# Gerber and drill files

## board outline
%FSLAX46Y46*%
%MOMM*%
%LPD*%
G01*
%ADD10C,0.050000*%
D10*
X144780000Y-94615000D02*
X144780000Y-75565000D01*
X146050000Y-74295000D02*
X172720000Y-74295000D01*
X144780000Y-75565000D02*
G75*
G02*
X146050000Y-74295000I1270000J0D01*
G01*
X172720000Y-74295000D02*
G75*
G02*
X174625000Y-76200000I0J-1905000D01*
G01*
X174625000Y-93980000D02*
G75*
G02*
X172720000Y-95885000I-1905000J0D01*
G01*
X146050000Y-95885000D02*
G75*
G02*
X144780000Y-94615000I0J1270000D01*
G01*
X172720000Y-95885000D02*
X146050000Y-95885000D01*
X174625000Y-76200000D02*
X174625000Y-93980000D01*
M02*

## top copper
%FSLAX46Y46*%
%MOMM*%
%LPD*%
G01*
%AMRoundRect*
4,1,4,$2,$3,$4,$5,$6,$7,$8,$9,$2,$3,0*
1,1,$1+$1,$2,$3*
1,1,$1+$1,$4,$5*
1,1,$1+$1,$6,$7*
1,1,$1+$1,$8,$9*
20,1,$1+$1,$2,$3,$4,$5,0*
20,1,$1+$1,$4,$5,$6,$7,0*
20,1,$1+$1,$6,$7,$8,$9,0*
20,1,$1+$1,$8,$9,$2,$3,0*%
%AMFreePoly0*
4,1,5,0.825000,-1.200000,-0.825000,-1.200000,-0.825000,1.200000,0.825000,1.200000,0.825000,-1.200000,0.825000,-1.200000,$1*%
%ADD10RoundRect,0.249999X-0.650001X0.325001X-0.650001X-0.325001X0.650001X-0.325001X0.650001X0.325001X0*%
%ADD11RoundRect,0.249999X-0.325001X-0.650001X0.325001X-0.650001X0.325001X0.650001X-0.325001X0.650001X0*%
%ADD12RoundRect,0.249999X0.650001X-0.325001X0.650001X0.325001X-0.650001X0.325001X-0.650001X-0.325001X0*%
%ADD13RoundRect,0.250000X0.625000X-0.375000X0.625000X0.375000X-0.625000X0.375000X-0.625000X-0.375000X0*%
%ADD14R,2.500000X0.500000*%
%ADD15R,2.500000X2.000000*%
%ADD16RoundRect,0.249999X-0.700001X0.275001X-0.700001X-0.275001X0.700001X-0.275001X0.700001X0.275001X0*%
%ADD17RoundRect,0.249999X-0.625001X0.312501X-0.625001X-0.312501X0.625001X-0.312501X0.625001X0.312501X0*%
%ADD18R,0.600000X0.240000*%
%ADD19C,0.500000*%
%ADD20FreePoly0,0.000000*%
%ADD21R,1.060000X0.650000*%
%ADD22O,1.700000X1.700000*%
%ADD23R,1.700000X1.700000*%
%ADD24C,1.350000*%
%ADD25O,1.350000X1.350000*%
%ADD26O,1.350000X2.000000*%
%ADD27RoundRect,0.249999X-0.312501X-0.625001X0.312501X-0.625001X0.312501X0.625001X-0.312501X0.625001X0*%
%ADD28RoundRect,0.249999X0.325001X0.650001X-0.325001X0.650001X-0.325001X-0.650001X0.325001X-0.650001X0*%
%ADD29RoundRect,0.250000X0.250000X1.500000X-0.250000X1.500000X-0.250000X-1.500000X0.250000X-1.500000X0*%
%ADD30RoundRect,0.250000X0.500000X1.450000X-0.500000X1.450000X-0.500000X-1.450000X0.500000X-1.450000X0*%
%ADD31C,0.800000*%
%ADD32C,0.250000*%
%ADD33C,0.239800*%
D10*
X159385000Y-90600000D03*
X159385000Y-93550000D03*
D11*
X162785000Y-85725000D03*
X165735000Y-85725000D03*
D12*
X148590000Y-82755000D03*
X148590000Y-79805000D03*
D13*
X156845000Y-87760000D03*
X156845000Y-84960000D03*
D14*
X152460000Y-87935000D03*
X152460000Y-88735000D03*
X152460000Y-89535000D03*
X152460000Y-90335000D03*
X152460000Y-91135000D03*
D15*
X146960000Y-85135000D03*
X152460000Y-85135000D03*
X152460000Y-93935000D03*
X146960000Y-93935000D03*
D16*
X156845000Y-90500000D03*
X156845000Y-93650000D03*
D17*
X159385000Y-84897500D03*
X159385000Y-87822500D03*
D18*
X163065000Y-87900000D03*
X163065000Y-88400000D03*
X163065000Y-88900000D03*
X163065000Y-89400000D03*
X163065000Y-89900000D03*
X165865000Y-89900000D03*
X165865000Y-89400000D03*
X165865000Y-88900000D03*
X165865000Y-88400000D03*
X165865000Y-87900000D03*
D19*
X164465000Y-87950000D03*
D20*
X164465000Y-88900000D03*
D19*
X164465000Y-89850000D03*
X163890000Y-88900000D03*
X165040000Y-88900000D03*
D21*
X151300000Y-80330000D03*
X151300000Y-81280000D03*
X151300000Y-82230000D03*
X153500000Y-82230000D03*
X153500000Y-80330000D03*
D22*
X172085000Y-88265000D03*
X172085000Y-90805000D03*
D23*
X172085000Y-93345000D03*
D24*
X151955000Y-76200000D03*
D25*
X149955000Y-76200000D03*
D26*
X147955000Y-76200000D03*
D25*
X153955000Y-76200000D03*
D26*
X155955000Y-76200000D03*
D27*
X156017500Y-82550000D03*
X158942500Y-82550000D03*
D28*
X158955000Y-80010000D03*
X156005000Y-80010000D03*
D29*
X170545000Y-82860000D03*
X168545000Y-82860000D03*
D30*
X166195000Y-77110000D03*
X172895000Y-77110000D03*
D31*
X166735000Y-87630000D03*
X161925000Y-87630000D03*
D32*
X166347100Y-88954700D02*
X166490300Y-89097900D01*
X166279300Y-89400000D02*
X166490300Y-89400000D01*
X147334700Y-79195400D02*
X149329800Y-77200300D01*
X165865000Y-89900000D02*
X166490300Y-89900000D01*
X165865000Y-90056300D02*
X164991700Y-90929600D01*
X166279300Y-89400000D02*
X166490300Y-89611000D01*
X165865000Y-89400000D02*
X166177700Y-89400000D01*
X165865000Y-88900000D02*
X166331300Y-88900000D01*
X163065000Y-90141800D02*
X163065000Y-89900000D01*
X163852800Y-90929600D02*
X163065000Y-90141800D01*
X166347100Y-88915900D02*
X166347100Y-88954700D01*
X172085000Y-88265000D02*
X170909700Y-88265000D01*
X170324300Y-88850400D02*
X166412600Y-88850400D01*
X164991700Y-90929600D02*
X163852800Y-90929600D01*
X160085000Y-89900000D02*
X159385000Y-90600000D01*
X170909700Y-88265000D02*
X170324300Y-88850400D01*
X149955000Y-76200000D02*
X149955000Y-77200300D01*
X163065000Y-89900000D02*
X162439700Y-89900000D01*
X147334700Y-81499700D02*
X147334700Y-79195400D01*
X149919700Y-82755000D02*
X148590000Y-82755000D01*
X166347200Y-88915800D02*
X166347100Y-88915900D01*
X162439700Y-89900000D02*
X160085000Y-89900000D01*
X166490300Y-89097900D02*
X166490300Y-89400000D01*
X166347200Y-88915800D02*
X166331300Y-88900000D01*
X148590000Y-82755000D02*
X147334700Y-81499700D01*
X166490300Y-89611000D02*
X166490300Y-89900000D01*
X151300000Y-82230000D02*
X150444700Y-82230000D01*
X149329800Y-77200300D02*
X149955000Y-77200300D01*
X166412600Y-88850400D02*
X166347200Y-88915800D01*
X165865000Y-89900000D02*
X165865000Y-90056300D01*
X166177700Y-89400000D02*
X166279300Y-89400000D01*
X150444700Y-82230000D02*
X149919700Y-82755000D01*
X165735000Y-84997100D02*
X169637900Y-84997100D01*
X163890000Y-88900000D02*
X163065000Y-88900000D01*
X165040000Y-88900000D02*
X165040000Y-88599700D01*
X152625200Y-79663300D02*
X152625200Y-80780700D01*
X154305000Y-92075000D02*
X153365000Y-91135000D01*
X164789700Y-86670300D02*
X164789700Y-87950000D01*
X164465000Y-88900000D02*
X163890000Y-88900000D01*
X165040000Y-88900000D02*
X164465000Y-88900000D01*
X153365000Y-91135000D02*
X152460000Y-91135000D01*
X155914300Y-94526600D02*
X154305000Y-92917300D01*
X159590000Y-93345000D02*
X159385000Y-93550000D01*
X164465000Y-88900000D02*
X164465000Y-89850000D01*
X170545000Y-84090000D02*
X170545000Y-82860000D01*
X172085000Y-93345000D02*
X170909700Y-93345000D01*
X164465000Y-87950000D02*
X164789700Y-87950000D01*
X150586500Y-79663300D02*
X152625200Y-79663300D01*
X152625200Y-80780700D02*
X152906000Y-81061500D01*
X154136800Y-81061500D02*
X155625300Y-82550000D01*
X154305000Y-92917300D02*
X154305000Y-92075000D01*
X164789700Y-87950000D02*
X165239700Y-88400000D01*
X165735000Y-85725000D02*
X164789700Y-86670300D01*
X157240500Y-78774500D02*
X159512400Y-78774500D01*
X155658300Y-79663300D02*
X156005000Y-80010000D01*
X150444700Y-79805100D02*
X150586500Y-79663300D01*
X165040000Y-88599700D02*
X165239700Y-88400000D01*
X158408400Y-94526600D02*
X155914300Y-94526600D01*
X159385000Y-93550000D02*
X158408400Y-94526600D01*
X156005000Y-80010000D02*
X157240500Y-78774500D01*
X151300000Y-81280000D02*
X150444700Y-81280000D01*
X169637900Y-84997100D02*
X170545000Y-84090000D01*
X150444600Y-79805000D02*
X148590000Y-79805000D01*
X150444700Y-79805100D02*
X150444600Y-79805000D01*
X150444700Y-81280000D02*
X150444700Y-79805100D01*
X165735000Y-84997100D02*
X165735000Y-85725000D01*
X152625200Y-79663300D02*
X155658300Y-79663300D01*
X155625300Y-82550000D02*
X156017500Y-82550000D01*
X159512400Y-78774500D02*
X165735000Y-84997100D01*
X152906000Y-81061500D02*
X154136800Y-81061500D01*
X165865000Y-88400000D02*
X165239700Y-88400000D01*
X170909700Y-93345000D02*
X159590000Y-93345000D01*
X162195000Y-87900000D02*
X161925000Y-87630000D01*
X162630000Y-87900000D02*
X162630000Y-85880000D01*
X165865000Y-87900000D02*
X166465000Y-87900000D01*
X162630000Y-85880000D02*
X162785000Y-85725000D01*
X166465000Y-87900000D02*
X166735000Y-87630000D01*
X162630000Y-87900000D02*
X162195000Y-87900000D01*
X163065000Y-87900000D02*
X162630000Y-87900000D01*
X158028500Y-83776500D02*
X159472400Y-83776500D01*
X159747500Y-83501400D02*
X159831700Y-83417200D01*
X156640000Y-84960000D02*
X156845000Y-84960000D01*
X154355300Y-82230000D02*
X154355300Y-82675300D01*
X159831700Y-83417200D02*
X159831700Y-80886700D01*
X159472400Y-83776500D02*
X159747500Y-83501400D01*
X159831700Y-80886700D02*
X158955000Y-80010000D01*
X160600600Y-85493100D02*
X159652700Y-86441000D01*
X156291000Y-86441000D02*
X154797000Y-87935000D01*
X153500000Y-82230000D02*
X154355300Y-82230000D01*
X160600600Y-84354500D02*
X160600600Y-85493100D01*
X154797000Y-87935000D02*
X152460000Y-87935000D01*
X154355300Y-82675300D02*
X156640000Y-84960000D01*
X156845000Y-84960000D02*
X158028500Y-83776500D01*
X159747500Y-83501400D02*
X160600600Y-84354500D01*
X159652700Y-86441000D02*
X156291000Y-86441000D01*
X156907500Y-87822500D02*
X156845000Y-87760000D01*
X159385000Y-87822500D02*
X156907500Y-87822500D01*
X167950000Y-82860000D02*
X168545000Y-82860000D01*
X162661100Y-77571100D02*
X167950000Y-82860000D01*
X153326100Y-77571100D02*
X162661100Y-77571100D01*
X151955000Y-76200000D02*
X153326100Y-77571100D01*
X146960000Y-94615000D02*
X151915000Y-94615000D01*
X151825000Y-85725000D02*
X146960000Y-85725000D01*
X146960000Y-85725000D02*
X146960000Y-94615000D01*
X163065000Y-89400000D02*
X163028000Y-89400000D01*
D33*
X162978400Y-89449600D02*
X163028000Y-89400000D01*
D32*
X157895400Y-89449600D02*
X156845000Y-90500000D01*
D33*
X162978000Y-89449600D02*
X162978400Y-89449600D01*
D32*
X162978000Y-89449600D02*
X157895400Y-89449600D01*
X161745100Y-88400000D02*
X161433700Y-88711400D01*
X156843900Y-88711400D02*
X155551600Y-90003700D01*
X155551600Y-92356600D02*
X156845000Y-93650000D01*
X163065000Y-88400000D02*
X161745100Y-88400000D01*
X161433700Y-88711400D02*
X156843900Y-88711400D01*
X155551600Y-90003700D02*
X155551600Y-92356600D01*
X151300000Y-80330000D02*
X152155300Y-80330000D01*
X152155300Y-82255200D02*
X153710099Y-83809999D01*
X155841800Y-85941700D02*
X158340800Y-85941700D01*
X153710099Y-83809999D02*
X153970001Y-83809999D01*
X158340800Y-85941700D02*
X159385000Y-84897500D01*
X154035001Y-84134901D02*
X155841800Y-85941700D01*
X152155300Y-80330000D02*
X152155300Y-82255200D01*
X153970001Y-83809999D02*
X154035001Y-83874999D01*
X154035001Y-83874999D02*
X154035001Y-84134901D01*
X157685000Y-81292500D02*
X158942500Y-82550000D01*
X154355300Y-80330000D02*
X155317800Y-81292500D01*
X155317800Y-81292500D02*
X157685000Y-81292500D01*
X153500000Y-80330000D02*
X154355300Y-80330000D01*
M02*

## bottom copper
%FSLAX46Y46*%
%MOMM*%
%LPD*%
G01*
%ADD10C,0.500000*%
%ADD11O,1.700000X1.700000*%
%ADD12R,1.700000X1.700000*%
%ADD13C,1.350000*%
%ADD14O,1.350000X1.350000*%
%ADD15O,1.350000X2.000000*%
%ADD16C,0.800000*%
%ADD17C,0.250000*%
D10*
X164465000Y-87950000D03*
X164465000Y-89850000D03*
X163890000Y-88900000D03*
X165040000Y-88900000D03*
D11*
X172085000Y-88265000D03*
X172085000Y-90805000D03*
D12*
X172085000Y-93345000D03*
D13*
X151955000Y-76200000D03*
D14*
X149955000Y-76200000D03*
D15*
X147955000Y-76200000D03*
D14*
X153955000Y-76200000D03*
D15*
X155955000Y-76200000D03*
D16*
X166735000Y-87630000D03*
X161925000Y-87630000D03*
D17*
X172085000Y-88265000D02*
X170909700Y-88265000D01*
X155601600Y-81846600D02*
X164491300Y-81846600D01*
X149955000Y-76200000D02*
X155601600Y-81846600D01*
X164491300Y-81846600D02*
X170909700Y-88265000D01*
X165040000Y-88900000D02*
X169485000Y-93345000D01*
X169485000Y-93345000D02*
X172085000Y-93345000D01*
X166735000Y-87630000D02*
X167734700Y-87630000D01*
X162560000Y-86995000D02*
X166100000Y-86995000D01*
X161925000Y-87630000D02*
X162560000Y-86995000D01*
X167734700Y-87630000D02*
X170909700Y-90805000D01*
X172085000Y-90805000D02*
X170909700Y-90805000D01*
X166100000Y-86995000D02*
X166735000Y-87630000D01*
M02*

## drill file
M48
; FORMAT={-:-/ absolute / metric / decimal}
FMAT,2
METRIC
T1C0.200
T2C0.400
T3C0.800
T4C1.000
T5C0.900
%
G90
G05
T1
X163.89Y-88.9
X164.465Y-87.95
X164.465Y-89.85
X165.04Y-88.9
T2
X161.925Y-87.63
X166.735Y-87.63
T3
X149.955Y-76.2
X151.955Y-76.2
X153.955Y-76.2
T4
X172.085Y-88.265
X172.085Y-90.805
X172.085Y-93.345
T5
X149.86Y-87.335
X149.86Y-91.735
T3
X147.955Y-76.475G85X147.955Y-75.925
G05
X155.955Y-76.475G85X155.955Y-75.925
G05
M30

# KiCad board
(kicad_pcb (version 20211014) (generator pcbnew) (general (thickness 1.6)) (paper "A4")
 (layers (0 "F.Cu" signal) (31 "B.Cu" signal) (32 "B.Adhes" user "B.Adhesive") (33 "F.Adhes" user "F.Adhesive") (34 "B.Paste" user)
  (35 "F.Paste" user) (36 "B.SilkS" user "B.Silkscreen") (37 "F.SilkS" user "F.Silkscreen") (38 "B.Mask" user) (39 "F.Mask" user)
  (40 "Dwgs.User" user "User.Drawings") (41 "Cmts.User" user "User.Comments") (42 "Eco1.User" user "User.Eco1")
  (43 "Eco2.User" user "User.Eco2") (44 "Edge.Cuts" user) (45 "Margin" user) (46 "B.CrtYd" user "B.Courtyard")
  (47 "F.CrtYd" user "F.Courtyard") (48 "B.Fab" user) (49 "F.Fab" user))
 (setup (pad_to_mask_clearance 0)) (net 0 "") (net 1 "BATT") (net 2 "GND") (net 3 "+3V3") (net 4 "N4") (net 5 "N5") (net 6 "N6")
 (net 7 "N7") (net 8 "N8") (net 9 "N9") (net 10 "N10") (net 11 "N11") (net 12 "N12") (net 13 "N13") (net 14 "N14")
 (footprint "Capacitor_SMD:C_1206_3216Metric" (layer "F.Cu") (at 159.385 92.075 -90)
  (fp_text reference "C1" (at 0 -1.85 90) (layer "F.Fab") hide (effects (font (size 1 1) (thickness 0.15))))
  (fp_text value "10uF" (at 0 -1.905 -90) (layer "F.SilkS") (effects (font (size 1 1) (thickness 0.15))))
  (pad "1" smd roundrect locked (at -1.475 0 270) (size 1.15 1.8) (layers "F.Cu" "F.Paste" "F.Mask") (roundrect_rratio 0.2173904348)
   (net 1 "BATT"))
  (pad "2" smd roundrect locked (at 1.475 0 270) (size 1.15 1.8) (layers "F.Cu" "F.Paste" "F.Mask") (roundrect_rratio 0.2173904348)
   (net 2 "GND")))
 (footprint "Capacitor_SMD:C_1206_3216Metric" (layer "F.Cu") (at 164.26 85.725)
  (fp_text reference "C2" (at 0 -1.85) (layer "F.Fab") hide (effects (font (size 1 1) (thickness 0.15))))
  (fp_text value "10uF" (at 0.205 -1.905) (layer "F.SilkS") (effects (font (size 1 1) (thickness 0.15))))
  (pad "1" smd roundrect locked (at -1.475 0) (size 1.15 1.8) (layers "F.Cu" "F.Paste" "F.Mask") (roundrect_rratio 0.2173904348)
   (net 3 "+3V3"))
  (pad "2" smd roundrect locked (at 1.475 0) (size 1.15 1.8) (layers "F.Cu" "F.Paste" "F.Mask") (roundrect_rratio 0.2173904348)
   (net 2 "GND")))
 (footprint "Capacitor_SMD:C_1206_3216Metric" (layer "F.Cu") (at 148.59 81.28 90)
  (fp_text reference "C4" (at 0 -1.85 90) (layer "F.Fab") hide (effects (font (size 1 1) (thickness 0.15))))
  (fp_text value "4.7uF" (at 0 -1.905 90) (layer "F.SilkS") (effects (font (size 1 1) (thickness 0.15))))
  (pad "1" smd roundrect locked (at -1.475 0 90) (size 1.15 1.8) (layers "F.Cu" "F.Paste" "F.Mask") (roundrect_rratio 0.2173904348)
   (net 1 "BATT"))
  (pad "2" smd roundrect locked (at 1.475 0 90) (size 1.15 1.8) (layers "F.Cu" "F.Paste" "F.Mask") (roundrect_rratio 0.2173904348)
   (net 2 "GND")))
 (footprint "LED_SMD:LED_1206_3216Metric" (layer "F.Cu") (at 156.845 86.36 90)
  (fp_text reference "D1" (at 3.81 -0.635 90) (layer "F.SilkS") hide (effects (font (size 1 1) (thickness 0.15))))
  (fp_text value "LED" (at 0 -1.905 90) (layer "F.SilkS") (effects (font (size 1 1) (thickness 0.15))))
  (pad "1" smd roundrect locked (at -1.4 0 90) (size 1.25 1.75) (layers "F.Cu" "F.Paste" "F.Mask") (roundrect_rratio 0.2) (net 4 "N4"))
  (pad "2" smd roundrect locked (at 1.4 0 90) (size 1.25 1.75) (layers "F.Cu" "F.Paste" "F.Mask") (roundrect_rratio 0.2) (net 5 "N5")))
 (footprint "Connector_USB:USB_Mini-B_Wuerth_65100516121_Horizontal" (layer "F.Cu") (at 149.86 89.535 -90)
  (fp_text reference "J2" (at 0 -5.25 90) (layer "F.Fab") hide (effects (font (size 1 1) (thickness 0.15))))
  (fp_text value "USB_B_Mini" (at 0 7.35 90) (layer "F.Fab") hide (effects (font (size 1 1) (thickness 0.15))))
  (pad "" np_thru_hole circle locked (at 2.2 0 270) (size 0.9 0.9) (drill 0.9) (layers *.Cu *.Mask))
  (pad "" np_thru_hole circle locked (at -2.2 0 270) (size 0.9 0.9) (drill 0.9) (layers *.Cu *.Mask))
  (pad "1" smd rect locked (at -1.6 -2.6 270) (size 0.5 2.5) (layers "F.Cu" "F.Paste" "F.Mask") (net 5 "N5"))
  (pad "2" smd rect locked (at -0.8 -2.6 270) (size 0.5 2.5) (layers "F.Cu" "F.Paste" "F.Mask") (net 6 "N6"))
  (pad "3" smd rect locked (at 0 -2.6 270) (size 0.5 2.5) (layers "F.Cu" "F.Paste" "F.Mask") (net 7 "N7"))
  (pad "4" smd rect locked (at 0.8 -2.6 270) (size 0.5 2.5) (layers "F.Cu" "F.Paste" "F.Mask") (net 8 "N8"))
  (pad "5" smd rect locked (at 1.6 -2.6 270) (size 0.5 2.5) (layers "F.Cu" "F.Paste" "F.Mask") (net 2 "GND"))
  (pad "6" smd rect locked (at -4.4 2.9 270) (size 2 2.5) (layers "F.Cu" "F.Paste" "F.Mask") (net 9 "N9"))
  (pad "6" smd rect locked (at -4.4 -2.6 270) (size 2 2.5) (layers "F.Cu" "F.Paste" "F.Mask") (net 9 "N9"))
  (pad "6" smd rect locked (at 4.4 -2.6 270) (size 2 2.5) (layers "F.Cu" "F.Paste" "F.Mask") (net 9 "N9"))
  (pad "6" smd rect locked (at 4.4 2.9 270) (size 2 2.5) (layers "F.Cu" "F.Paste" "F.Mask") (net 9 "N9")))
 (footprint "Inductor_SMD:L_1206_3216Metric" (layer "F.Cu") (at 156.845 92.075 -90)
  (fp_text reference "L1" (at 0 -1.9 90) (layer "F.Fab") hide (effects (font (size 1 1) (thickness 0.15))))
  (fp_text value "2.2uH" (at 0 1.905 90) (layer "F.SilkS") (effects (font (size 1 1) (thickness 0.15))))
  (pad "1" smd roundrect locked (at -1.575 0 270) (size 1.05 1.9) (layers "F.Cu" "F.Paste" "F.Mask") (roundrect_rratio 0.2380942857)
   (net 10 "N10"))
  (pad "2" smd roundrect locked (at 1.575 0 270) (size 1.05 1.9) (layers "F.Cu" "F.Paste" "F.Mask") (roundrect_rratio 0.2380942857)
   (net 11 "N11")))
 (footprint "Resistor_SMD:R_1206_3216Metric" (layer "F.Cu") (at 159.385 86.36 -90)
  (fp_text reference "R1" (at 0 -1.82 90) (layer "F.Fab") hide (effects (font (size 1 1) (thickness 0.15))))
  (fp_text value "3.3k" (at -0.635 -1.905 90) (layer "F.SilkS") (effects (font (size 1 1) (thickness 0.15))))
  (pad "1" smd roundrect locked (at -1.4625 0 270) (size 1.125 1.75) (layers "F.Cu" "F.Paste" "F.Mask") (roundrect_rratio 0.2222213333)
   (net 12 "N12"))
  (pad "2" smd roundrect locked (at 1.4625 0 270) (size 1.125 1.75) (layers "F.Cu" "F.Paste" "F.Mask") (roundrect_rratio 0.2222213333)
   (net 4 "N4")))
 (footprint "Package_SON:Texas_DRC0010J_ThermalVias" (layer "F.Cu") (at 164.465 88.9)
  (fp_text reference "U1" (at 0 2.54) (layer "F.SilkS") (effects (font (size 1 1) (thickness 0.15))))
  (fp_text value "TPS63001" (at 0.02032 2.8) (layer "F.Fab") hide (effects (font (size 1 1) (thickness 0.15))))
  (pad "" smd roundrect locked (at 0.25 -1.53) (size 0.25 0.34) (layers "F.Paste") (roundrect_rratio 0.1) (zone_connect 0))
  (pad "" smd roundrect locked (at -0.25 1.53) (size 0.25 0.34) (layers "F.Paste") (roundrect_rratio 0.1) (zone_connect 0))
  (pad "" smd roundrect locked (at -0.25 -1.53) (size 0.25 0.34) (layers "F.Paste") (roundrect_rratio 0.1) (zone_connect 0))
  (pad "" smd roundrect locked (at 0 -0.63) (size 1.5 1.06) (layers "F.Paste") (roundrect_rratio 0.1) (zone_connect 0))
  (pad "" smd roundrect locked (at 0 0.63) (size 1.5 1.06) (layers "F.Paste") (roundrect_rratio 0.1) (zone_connect 0))
  (pad "" smd roundrect locked (at 0.25 1.53) (size 0.25 0.34) (layers "F.Paste") (roundrect_rratio 0.1) (zone_connect 0))
  (pad "1" smd rect locked (at -1.4 -1) (size 0.6 0.24) (layers "F.Cu" "F.Paste" "F.Mask") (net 3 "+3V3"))
  (pad "2" smd rect locked (at -1.4 -0.5) (size 0.6 0.24) (layers "F.Cu" "F.Paste" "F.Mask") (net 11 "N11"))
  (pad "3" smd rect locked (at -1.4 0) (size 0.6 0.24) (layers "F.Cu" "F.Paste" "F.Mask") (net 2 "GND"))
  (pad "4" smd rect locked (at -1.4 0.5) (size 0.6 0.24) (layers "F.Cu" "F.Paste" "F.Mask") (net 10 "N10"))
  (pad "5" smd rect locked (at -1.4 1) (size 0.6 0.24) (layers "F.Cu" "F.Paste" "F.Mask") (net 1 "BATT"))
  (pad "6" smd rect locked (at 1.4 1) (size 0.6 0.24) (layers "F.Cu" "F.Paste" "F.Mask") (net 1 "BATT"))
  (pad "7" smd rect locked (at 1.4 0.5) (size 0.6 0.24) (layers "F.Cu" "F.Paste" "F.Mask") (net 1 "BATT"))
  (pad "8" smd rect locked (at 1.4 0) (size 0.6 0.24) (layers "F.Cu" "F.Paste" "F.Mask") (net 1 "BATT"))
  (pad "9" smd rect locked (at 1.4 -0.5) (size 0.6 0.24) (layers "F.Cu" "F.Paste" "F.Mask") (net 2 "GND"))
  (pad "10" smd rect locked (at 1.4 -1) (size 0.6 0.24) (layers "F.Cu" "F.Paste" "F.Mask") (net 3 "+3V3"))
  (pad "11" thru_hole circle locked (at 0 -0.95) (size 0.5 0.5) (drill 0.2) (layers *.Cu) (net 2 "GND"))
  (pad "11" smd custom locked (at 0 0) (size 1.65 2.4) (layers "F.Cu" "F.Mask") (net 2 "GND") (zone_connect 0)
   (options (clearance outline) (anchor rect)) (primitives))
  (pad "11" thru_hole circle locked (at 0 0.95) (size 0.5 0.5) (drill 0.2) (layers *.Cu) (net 2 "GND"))
  (pad "11" thru_hole circle locked (at -0.575 0) (size 0.5 0.5) (drill 0.2) (layers *.Cu) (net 2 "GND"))
  (pad "11" thru_hole circle locked (at 0.575 0) (size 0.5 0.5) (drill 0.2) (layers *.Cu) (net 2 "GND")))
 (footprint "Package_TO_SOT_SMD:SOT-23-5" (layer "F.Cu") (at 152.4 81.28)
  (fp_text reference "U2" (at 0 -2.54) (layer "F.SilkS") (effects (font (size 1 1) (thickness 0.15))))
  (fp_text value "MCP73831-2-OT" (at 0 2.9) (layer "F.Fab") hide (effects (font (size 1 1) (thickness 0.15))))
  (pad "1" smd rect locked (at -1.1 -0.95) (size 1.06 0.65) (layers "F.Cu" "F.Paste" "F.Mask") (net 12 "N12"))
  (pad "2" smd rect locked (at -1.1 0) (size 1.06 0.65) (layers "F.Cu" "F.Paste" "F.Mask") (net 2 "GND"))
  (pad "3" smd rect locked (at -1.1 0.95) (size 1.06 0.65) (layers "F.Cu" "F.Paste" "F.Mask") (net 1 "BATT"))
  (pad "4" smd rect locked (at 1.1 0.95) (size 1.06 0.65) (layers "F.Cu" "F.Paste" "F.Mask") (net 5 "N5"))
  (pad "5" smd rect locked (at 1.1 -0.95) (size 1.06 0.65) (layers "F.Cu" "F.Paste" "F.Mask") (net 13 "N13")))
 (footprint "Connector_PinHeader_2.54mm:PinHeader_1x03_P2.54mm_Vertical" (layer "F.Cu") (at 172.085 88.265)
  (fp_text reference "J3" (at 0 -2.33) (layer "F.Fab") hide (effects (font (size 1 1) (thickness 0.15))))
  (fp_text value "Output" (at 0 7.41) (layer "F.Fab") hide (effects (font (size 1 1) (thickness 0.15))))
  (pad "1" thru_hole oval locked (at 0 0) (size 1.7 1.7) (drill 1) (layers *.Cu *.Mask) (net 1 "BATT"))
  (pad "2" thru_hole oval locked (at 0 2.54) (size 1.7 1.7) (drill 1) (layers *.Cu *.Mask) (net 3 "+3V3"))
  (pad "3" thru_hole rect locked (at 0 5.08) (size 1.7 1.7) (drill 1) (layers *.Cu *.Mask) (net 2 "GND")))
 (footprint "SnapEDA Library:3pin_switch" (layer "F.Cu") (at 147.955 76.2 90)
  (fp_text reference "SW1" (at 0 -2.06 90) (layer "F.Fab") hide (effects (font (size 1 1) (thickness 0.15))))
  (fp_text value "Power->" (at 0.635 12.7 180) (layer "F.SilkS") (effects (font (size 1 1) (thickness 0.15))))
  (pad "1" thru_hole circle locked (at 0 4 90) (size 1.35 1.35) (drill 0.8) (layers *.Cu *.Mask) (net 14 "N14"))
  (pad "2" thru_hole oval locked (at 0 2 90) (size 1.35 1.35) (drill 0.8) (layers *.Cu *.Mask) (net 1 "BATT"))
  (pad "3" thru_hole oval locked (at 0 0 90) (size 2 1.35) (drill oval 1.35 0.8) (layers *.Cu *.Mask))
  (pad "4" thru_hole oval locked (at 0 6 90) (size 1.35 1.35) (drill 0.8) (layers *.Cu *.Mask))
  (pad "5" thru_hole oval locked (at 0 8 90) (size 2 1.35) (drill oval 1.35 0.8) (layers *.Cu *.Mask)))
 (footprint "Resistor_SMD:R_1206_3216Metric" (layer "F.Cu") (at 157.48 82.55)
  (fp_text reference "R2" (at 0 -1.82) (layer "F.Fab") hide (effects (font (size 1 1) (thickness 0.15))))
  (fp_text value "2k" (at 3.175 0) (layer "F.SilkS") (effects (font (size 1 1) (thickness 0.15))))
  (pad "1" smd roundrect locked (at -1.4625 0) (size 1.125 1.75) (layers "F.Cu" "F.Paste" "F.Mask") (roundrect_rratio 0.2222213333)
   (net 2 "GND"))
  (pad "2" smd roundrect locked (at 1.4625 0) (size 1.125 1.75) (layers "F.Cu" "F.Paste" "F.Mask") (roundrect_rratio 0.2222213333)
   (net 13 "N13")))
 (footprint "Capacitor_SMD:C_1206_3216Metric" (layer "F.Cu") (at 157.48 80.01 180)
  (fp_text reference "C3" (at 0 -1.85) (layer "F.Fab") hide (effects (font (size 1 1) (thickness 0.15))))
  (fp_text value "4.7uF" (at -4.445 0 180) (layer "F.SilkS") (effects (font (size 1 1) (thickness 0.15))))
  (pad "1" smd roundrect locked (at -1.475 0 180) (size 1.15 1.8) (layers "F.Cu" "F.Paste" "F.Mask") (roundrect_rratio 0.2173904348)
   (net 5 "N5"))
  (pad "2" smd roundrect locked (at 1.475 0 180) (size 1.15 1.8) (layers "F.Cu" "F.Paste" "F.Mask") (roundrect_rratio 0.2173904348)
   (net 2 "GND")))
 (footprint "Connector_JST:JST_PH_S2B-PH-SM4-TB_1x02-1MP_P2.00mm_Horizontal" (layer "F.Cu") (at 169.545 80.01 180)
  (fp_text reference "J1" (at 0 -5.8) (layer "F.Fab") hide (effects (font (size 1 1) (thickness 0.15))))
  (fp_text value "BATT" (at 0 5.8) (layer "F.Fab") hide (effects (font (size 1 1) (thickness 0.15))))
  (pad "1" smd roundrect locked (at -1 -2.85 180) (size 1 3.5) (layers "F.Cu" "F.Paste" "F.Mask") (roundrect_rratio 0.25) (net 2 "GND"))
  (pad "2" smd roundrect locked (at 1 -2.85 180) (size 1 3.5) (layers "F.Cu" "F.Paste" "F.Mask") (roundrect_rratio 0.25) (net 14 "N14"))
  (pad "MP" smd roundrect locked (at 3.35 2.9 180) (size 1.5 3.4) (layers "F.Cu" "F.Paste" "F.Mask") (roundrect_rratio 0.1666666667))
  (pad "MP" smd roundrect locked (at -3.35 2.9 180) (size 1.5 3.4) (layers "F.Cu" "F.Paste" "F.Mask") (roundrect_rratio 0.1666666667)))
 (gr_line (start 144.78 94.615) (end 144.78 75.565) (layer "Edge.Cuts") (width 0.05))
 (gr_line (start 146.05 74.295) (end 172.72 74.295) (layer "Edge.Cuts") (width 0.05))
 (gr_arc (start 144.78 75.565) (mid 145.151974 74.666974) (end 146.05 74.295) (layer "Edge.Cuts") (width 0.05))
 (gr_arc (start 172.72 74.295) (mid 174.067038 74.852962) (end 174.625 76.2) (layer "Edge.Cuts") (width 0.05))
 (gr_arc (start 174.625 93.98) (mid 174.067038 95.327038) (end 172.72 95.885) (layer "Edge.Cuts") (width 0.05))
 (gr_arc (start 146.05 95.885) (mid 145.151974 95.513026) (end 144.78 94.615) (layer "Edge.Cuts") (width 0.05))
 (gr_line (start 172.72 95.885) (end 146.05 95.885) (layer "Edge.Cuts") (width 0.05))
 (gr_line (start 174.625 76.2) (end 174.625 93.98) (layer "Edge.Cuts") (width 0.05))
 (segment (start 166.3471 88.9547) (end 166.4903 89.0979) (width 0.25) (layer "F.Cu") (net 1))
 (segment (start 166.2793 89.4) (end 166.4903 89.4) (width 0.25) (layer "F.Cu") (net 1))
 (segment (start 147.3347 79.1954) (end 149.3298 77.2003) (width 0.25) (layer "F.Cu") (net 1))
 (segment (start 165.865 89.9) (end 166.4903 89.9) (width 0.25) (layer "F.Cu") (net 1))
 (segment (start 165.865 90.0563) (end 164.9917 90.9296) (width 0.25) (layer "F.Cu") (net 1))
 (segment (start 166.2793 89.4) (end 166.4903 89.611) (width 0.25) (layer "F.Cu") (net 1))
 (segment (start 165.865 89.4) (end 166.1777 89.4) (width 0.25) (layer "F.Cu") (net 1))
 (segment (start 165.865 88.9) (end 166.3313 88.9) (width 0.25) (layer "F.Cu") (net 1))
 (segment (start 163.065 90.1418) (end 163.065 89.9) (width 0.25) (layer "F.Cu") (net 1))
 (segment (start 163.8528 90.9296) (end 163.065 90.1418) (width 0.25) (layer "F.Cu") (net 1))
 (segment (start 166.3471 88.9159) (end 166.3471 88.9547) (width 0.25) (layer "F.Cu") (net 1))
 (segment (start 172.085 88.265) (end 170.9097 88.265) (width 0.25) (layer "F.Cu") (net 1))
 (segment (start 170.3243 88.8504) (end 166.4126 88.8504) (width 0.25) (layer "F.Cu") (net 1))
 (segment (start 164.9917 90.9296) (end 163.8528 90.9296) (width 0.25) (layer "F.Cu") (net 1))
 (segment (start 160.085 89.9) (end 159.385 90.6) (width 0.25) (layer "F.Cu") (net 1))
 (segment (start 170.9097 88.265) (end 170.3243 88.8504) (width 0.25) (layer "F.Cu") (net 1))
 (segment (start 149.955 76.2) (end 149.955 77.2003) (width 0.25) (layer "F.Cu") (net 1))
 (segment (start 163.065 89.9) (end 162.4397 89.9) (width 0.25) (layer "F.Cu") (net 1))
 (segment (start 147.3347 81.4997) (end 147.3347 79.1954) (width 0.25) (layer "F.Cu") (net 1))
 (segment (start 149.9197 82.755) (end 148.59 82.755) (width 0.25) (layer "F.Cu") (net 1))
 (segment (start 166.3472 88.9158) (end 166.3471 88.9159) (width 0.25) (layer "F.Cu") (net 1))
 (segment (start 162.4397 89.9) (end 160.085 89.9) (width 0.25) (layer "F.Cu") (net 1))
 (segment (start 166.4903 89.0979) (end 166.4903 89.4) (width 0.25) (layer "F.Cu") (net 1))
 (segment (start 166.3472 88.9158) (end 166.3313 88.9) (width 0.25) (layer "F.Cu") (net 1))
 (segment (start 148.59 82.755) (end 147.3347 81.4997) (width 0.25) (layer "F.Cu") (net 1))
 (segment (start 166.4903 89.611) (end 166.4903 89.9) (width 0.25) (layer "F.Cu") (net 1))
 (segment (start 151.3 82.23) (end 150.4447 82.23) (width 0.25) (layer "F.Cu") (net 1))
 (segment (start 149.3298 77.2003) (end 149.955 77.2003) (width 0.25) (layer "F.Cu") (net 1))
 (segment (start 166.4126 88.8504) (end 166.3472 88.9158) (width 0.25) (layer "F.Cu") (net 1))
 (segment (start 165.865 89.9) (end 165.865 90.0563) (width 0.25) (layer "F.Cu") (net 1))
 (segment (start 166.1777 89.4) (end 166.2793 89.4) (width 0.25) (layer "F.Cu") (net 1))
 (segment (start 150.4447 82.23) (end 149.9197 82.755) (width 0.25) (layer "F.Cu") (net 1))
 (segment (start 172.085 88.265) (end 170.9097 88.265) (width 0.25) (layer "B.Cu") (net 1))
 (segment (start 155.6016 81.8466) (end 164.4913 81.8466) (width 0.25) (layer "B.Cu") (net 1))
 (segment (start 149.955 76.2) (end 155.6016 81.8466) (width 0.25) (layer "B.Cu") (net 1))
 (segment (start 164.4913 81.8466) (end 170.9097 88.265) (width 0.25) (layer "B.Cu") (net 1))
 (segment (start 165.735 84.9971) (end 169.6379 84.9971) (width 0.25) (layer "F.Cu") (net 2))
 (segment (start 163.89 88.9) (end 163.065 88.9) (width 0.25) (layer "F.Cu") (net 2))
 (segment (start 165.04 88.9) (end 165.04 88.5997) (width 0.25) (layer "F.Cu") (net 2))
 (segment (start 152.6252 79.6633) (end 152.6252 80.7807) (width 0.25) (layer "F.Cu") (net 2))
 (segment (start 154.305 92.075) (end 153.365 91.135) (width 0.25) (layer "F.Cu") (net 2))
 (segment (start 164.7897 86.6703) (end 164.7897 87.95) (width 0.25) (layer "F.Cu") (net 2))
 (segment (start 164.465 88.9) (end 163.89 88.9) (width 0.25) (layer "F.Cu") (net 2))
 (segment (start 165.04 88.9) (end 164.465 88.9) (width 0.25) (layer "F.Cu") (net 2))
 (segment (start 153.365 91.135) (end 152.46 91.135) (width 0.25) (layer "F.Cu") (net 2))
 (segment (start 155.9143 94.5266) (end 154.305 92.9173) (width 0.25) (layer "F.Cu") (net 2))
 (segment (start 159.59 93.345) (end 159.385 93.55) (width 0.25) (layer "F.Cu") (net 2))
 (segment (start 164.465 88.9) (end 164.465 89.85) (width 0.25) (layer "F.Cu") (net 2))
 (segment (start 170.545 84.09) (end 170.545 82.86) (width 0.25) (layer "F.Cu") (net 2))
 (segment (start 172.085 93.345) (end 170.9097 93.345) (width 0.25) (layer "F.Cu") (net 2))
 (segment (start 164.465 87.95) (end 164.7897 87.95) (width 0.25) (layer "F.Cu") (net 2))
 (segment (start 150.5865 79.6633) (end 152.6252 79.6633) (width 0.25) (layer "F.Cu") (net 2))
 (segment (start 152.6252 80.7807) (end 152.906 81.0615) (width 0.25) (layer "F.Cu") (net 2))
 (segment (start 154.1368 81.0615) (end 155.6253 82.55) (width 0.25) (layer "F.Cu") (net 2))
 (segment (start 154.305 92.9173) (end 154.305 92.075) (width 0.25) (layer "F.Cu") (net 2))
 (segment (start 164.7897 87.95) (end 165.2397 88.4) (width 0.25) (layer "F.Cu") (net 2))
 (segment (start 165.735 85.725) (end 164.7897 86.6703) (width 0.25) (layer "F.Cu") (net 2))
 (segment (start 157.2405 78.7745) (end 159.5124 78.7745) (width 0.25) (layer "F.Cu") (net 2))
 (segment (start 155.6583 79.6633) (end 156.005 80.01) (width 0.25) (layer "F.Cu") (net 2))
 (segment (start 150.4447 79.8051) (end 150.5865 79.6633) (width 0.25) (layer "F.Cu") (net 2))
 (segment (start 165.04 88.5997) (end 165.2397 88.4) (width 0.25) (layer "F.Cu") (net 2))
 (segment (start 158.4084 94.5266) (end 155.9143 94.5266) (width 0.25) (layer "F.Cu") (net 2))
 (segment (start 159.385 93.55) (end 158.4084 94.5266) (width 0.25) (layer "F.Cu") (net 2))
 (segment (start 156.005 80.01) (end 157.2405 78.7745) (width 0.25) (layer "F.Cu") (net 2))
 (segment (start 151.3 81.28) (end 150.4447 81.28) (width 0.25) (layer "F.Cu") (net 2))
 (segment (start 169.6379 84.9971) (end 170.545 84.09) (width 0.25) (layer "F.Cu") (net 2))
 (segment (start 150.4446 79.805) (end 148.59 79.805) (width 0.25) (layer "F.Cu") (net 2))
 (segment (start 150.4447 79.8051) (end 150.4446 79.805) (width 0.25) (layer "F.Cu") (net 2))
 (segment (start 150.4447 81.28) (end 150.4447 79.8051) (width 0.25) (layer "F.Cu") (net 2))
 (segment (start 165.735 84.9971) (end 165.735 85.725) (width 0.25) (layer "F.Cu") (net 2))
 (segment (start 152.6252 79.6633) (end 155.6583 79.6633) (width 0.25) (layer "F.Cu") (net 2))
 (segment (start 155.6253 82.55) (end 156.0175 82.55) (width 0.25) (layer "F.Cu") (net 2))
 (segment (start 159.5124 78.7745) (end 165.735 84.9971) (width 0.25) (layer "F.Cu") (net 2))
 (segment (start 152.906 81.0615) (end 154.1368 81.0615) (width 0.25) (layer "F.Cu") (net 2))
 (segment (start 165.865 88.4) (end 165.2397 88.4) (width 0.25) (layer "F.Cu") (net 2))
 (segment (start 170.9097 93.345) (end 159.59 93.345) (width 0.25) (layer "F.Cu") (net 2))
 (segment (start 165.04 88.9) (end 169.485 93.345) (width 0.25) (layer "B.Cu") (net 2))
 (segment (start 169.485 93.345) (end 172.085 93.345) (width 0.25) (layer "B.Cu") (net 2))
 (segment (start 162.195 87.9) (end 161.925 87.63) (width 0.25) (layer "F.Cu") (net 3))
 (segment (start 162.63 87.9) (end 162.63 85.88) (width 0.25) (layer "F.Cu") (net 3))
 (segment (start 165.865 87.9) (end 166.465 87.9) (width 0.25) (layer "F.Cu") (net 3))
 (segment (start 162.63 85.88) (end 162.785 85.725) (width 0.25) (layer "F.Cu") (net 3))
 (segment (start 166.465 87.9) (end 166.735 87.63) (width 0.25) (layer "F.Cu") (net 3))
 (segment (start 162.63 87.9) (end 162.195 87.9) (width 0.25) (layer "F.Cu") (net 3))
 (segment (start 163.065 87.9) (end 162.63 87.9) (width 0.25) (layer "F.Cu") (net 3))
 (via (at 166.735 87.63) (size 0.8) (drill 0.4) (layers "F.Cu" "B.Cu") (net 3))
 (via (at 161.925 87.63) (size 0.8) (drill 0.4) (layers "F.Cu" "B.Cu") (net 3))
 (segment (start 166.735 87.63) (end 167.7347 87.63) (width 0.25) (layer "B.Cu") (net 3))
 (segment (start 162.56 86.995) (end 166.1 86.995) (width 0.25) (layer "B.Cu") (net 3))
 (segment (start 161.925 87.63) (end 162.56 86.995) (width 0.25) (layer "B.Cu") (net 3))
 (segment (start 167.7347 87.63) (end 170.9097 90.805) (width 0.25) (layer "B.Cu") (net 3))
 (segment (start 172.085 90.805) (end 170.9097 90.805) (width 0.25) (layer "B.Cu") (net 3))
 (segment (start 166.1 86.995) (end 166.735 87.63) (width 0.25) (layer "B.Cu") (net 3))
 (segment (start 158.0285 83.7765) (end 159.4724 83.7765) (width 0.25) (layer "F.Cu") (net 5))
 (segment (start 159.7475 83.5014) (end 159.8317 83.4172) (width 0.25) (layer "F.Cu") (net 5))
 (segment (start 156.64 84.96) (end 156.845 84.96) (width 0.25) (layer "F.Cu") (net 5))
 (segment (start 154.3553 82.23) (end 154.3553 82.6753) (width 0.25) (layer "F.Cu") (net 5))
 (segment (start 159.8317 83.4172) (end 159.8317 80.8867) (width 0.25) (layer "F.Cu") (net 5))
 (segment (start 159.4724 83.7765) (end 159.7475 83.5014) (width 0.25) (layer "F.Cu") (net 5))
 (segment (start 159.8317 80.8867) (end 158.955 80.01) (width 0.25) (layer "F.Cu") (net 5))
 (segment (start 160.6006 85.4931) (end 159.6527 86.441) (width 0.25) (layer "F.Cu") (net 5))
 (segment (start 156.291 86.441) (end 154.797 87.935) (width 0.25) (layer "F.Cu") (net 5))
 (segment (start 153.5 82.23) (end 154.3553 82.23) (width 0.25) (layer "F.Cu") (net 5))
 (segment (start 160.6006 84.3545) (end 160.6006 85.4931) (width 0.25) (layer "F.Cu") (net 5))
 (segment (start 154.797 87.935) (end 152.46 87.935) (width 0.25) (layer "F.Cu") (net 5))
 (segment (start 154.3553 82.6753) (end 156.64 84.96) (width 0.25) (layer "F.Cu") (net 5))
 (segment (start 156.845 84.96) (end 158.0285 83.7765) (width 0.25) (layer "F.Cu") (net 5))
 (segment (start 159.7475 83.5014) (end 160.6006 84.3545) (width 0.25) (layer "F.Cu") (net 5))
 (segment (start 159.6527 86.441) (end 156.291 86.441) (width 0.25) (layer "F.Cu") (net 5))
 (segment (start 156.9075 87.8225) (end 156.845 87.76) (width 0.25) (layer "F.Cu") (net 4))
 (segment (start 159.385 87.8225) (end 156.9075 87.8225) (width 0.25) (layer "F.Cu") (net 4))
 (segment (start 167.95 82.86) (end 168.545 82.86) (width 0.25) (layer "F.Cu") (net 14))
 (segment (start 162.6611 77.5711) (end 167.95 82.86) (width 0.25) (layer "F.Cu") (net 14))
 (segment (start 153.3261 77.5711) (end 162.6611 77.5711) (width 0.25) (layer "F.Cu") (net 14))
 (segment (start 151.955 76.2) (end 153.3261 77.5711) (width 0.25) (layer "F.Cu") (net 14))
 (segment (start 146.96 94.615) (end 151.915 94.615) (width 0.25) (layer "F.Cu") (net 9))
 (segment (start 151.825 85.725) (end 146.96 85.725) (width 0.25) (layer "F.Cu") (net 9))
 (segment (start 146.96 85.725) (end 146.96 94.615) (width 0.25) (layer "F.Cu") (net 9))
 (segment (start 163.065 89.4) (end 163.028 89.4) (width 0.25) (layer "F.Cu") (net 10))
 (segment (start 162.9784 89.4496) (end 163.028 89.4) (width 0.2398) (layer "F.Cu") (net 10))
 (segment (start 157.8954 89.4496) (end 156.845 90.5) (width 0.25) (layer "F.Cu") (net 10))
 (segment (start 162.978 89.4496) (end 162.9784 89.4496) (width 0.2398) (layer "F.Cu") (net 10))
 (segment (start 162.978 89.4496) (end 157.8954 89.4496) (width 0.25) (layer "F.Cu") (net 10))
 (segment (start 161.7451 88.4) (end 161.4337 88.7114) (width 0.25) (layer "F.Cu") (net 11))
 (segment (start 156.8439 88.7114) (end 155.5516 90.0037) (width 0.25) (layer "F.Cu") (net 11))
 (segment (start 155.5516 92.3566) (end 156.845 93.65) (width 0.25) (layer "F.Cu") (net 11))
 (segment (start 163.065 88.4) (end 161.7451 88.4) (width 0.25) (layer "F.Cu") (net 11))
 (segment (start 161.4337 88.7114) (end 156.8439 88.7114) (width 0.25) (layer "F.Cu") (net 11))
 (segment (start 155.5516 90.0037) (end 155.5516 92.3566) (width 0.25) (layer "F.Cu") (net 11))
 (segment (start 151.3 80.33) (end 152.1553 80.33) (width 0.25) (layer "F.Cu") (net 12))
 (segment (start 152.1553 82.2552) (end 153.710099 83.809999) (width 0.25) (layer "F.Cu") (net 12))
 (segment (start 155.8418 85.9417) (end 158.3408 85.9417) (width 0.25) (layer "F.Cu") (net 12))
 (segment (start 153.710099 83.809999) (end 153.970001 83.809999) (width 0.25) (layer "F.Cu") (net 12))
 (segment (start 158.3408 85.9417) (end 159.385 84.8975) (width 0.25) (layer "F.Cu") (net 12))
 (segment (start 154.035001 84.134901) (end 155.8418 85.9417) (width 0.25) (layer "F.Cu") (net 12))
 (segment (start 152.1553 80.33) (end 152.1553 82.2552) (width 0.25) (layer "F.Cu") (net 12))
 (segment (start 153.970001 83.809999) (end 154.035001 83.874999) (width 0.25) (layer "F.Cu") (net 12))
 (segment (start 154.035001 83.874999) (end 154.035001 84.134901) (width 0.25) (layer "F.Cu") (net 12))
 (segment (start 157.685 81.2925) (end 158.9425 82.55) (width 0.25) (layer "F.Cu") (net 13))
 (segment (start 154.3553 80.33) (end 155.3178 81.2925) (width 0.25) (layer "F.Cu") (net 13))
 (segment (start 155.3178 81.2925) (end 157.685 81.2925) (width 0.25) (layer "F.Cu") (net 13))
 (segment (start 153.5 80.33) (end 154.3553 80.33) (width 0.25) (layer "F.Cu") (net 13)))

